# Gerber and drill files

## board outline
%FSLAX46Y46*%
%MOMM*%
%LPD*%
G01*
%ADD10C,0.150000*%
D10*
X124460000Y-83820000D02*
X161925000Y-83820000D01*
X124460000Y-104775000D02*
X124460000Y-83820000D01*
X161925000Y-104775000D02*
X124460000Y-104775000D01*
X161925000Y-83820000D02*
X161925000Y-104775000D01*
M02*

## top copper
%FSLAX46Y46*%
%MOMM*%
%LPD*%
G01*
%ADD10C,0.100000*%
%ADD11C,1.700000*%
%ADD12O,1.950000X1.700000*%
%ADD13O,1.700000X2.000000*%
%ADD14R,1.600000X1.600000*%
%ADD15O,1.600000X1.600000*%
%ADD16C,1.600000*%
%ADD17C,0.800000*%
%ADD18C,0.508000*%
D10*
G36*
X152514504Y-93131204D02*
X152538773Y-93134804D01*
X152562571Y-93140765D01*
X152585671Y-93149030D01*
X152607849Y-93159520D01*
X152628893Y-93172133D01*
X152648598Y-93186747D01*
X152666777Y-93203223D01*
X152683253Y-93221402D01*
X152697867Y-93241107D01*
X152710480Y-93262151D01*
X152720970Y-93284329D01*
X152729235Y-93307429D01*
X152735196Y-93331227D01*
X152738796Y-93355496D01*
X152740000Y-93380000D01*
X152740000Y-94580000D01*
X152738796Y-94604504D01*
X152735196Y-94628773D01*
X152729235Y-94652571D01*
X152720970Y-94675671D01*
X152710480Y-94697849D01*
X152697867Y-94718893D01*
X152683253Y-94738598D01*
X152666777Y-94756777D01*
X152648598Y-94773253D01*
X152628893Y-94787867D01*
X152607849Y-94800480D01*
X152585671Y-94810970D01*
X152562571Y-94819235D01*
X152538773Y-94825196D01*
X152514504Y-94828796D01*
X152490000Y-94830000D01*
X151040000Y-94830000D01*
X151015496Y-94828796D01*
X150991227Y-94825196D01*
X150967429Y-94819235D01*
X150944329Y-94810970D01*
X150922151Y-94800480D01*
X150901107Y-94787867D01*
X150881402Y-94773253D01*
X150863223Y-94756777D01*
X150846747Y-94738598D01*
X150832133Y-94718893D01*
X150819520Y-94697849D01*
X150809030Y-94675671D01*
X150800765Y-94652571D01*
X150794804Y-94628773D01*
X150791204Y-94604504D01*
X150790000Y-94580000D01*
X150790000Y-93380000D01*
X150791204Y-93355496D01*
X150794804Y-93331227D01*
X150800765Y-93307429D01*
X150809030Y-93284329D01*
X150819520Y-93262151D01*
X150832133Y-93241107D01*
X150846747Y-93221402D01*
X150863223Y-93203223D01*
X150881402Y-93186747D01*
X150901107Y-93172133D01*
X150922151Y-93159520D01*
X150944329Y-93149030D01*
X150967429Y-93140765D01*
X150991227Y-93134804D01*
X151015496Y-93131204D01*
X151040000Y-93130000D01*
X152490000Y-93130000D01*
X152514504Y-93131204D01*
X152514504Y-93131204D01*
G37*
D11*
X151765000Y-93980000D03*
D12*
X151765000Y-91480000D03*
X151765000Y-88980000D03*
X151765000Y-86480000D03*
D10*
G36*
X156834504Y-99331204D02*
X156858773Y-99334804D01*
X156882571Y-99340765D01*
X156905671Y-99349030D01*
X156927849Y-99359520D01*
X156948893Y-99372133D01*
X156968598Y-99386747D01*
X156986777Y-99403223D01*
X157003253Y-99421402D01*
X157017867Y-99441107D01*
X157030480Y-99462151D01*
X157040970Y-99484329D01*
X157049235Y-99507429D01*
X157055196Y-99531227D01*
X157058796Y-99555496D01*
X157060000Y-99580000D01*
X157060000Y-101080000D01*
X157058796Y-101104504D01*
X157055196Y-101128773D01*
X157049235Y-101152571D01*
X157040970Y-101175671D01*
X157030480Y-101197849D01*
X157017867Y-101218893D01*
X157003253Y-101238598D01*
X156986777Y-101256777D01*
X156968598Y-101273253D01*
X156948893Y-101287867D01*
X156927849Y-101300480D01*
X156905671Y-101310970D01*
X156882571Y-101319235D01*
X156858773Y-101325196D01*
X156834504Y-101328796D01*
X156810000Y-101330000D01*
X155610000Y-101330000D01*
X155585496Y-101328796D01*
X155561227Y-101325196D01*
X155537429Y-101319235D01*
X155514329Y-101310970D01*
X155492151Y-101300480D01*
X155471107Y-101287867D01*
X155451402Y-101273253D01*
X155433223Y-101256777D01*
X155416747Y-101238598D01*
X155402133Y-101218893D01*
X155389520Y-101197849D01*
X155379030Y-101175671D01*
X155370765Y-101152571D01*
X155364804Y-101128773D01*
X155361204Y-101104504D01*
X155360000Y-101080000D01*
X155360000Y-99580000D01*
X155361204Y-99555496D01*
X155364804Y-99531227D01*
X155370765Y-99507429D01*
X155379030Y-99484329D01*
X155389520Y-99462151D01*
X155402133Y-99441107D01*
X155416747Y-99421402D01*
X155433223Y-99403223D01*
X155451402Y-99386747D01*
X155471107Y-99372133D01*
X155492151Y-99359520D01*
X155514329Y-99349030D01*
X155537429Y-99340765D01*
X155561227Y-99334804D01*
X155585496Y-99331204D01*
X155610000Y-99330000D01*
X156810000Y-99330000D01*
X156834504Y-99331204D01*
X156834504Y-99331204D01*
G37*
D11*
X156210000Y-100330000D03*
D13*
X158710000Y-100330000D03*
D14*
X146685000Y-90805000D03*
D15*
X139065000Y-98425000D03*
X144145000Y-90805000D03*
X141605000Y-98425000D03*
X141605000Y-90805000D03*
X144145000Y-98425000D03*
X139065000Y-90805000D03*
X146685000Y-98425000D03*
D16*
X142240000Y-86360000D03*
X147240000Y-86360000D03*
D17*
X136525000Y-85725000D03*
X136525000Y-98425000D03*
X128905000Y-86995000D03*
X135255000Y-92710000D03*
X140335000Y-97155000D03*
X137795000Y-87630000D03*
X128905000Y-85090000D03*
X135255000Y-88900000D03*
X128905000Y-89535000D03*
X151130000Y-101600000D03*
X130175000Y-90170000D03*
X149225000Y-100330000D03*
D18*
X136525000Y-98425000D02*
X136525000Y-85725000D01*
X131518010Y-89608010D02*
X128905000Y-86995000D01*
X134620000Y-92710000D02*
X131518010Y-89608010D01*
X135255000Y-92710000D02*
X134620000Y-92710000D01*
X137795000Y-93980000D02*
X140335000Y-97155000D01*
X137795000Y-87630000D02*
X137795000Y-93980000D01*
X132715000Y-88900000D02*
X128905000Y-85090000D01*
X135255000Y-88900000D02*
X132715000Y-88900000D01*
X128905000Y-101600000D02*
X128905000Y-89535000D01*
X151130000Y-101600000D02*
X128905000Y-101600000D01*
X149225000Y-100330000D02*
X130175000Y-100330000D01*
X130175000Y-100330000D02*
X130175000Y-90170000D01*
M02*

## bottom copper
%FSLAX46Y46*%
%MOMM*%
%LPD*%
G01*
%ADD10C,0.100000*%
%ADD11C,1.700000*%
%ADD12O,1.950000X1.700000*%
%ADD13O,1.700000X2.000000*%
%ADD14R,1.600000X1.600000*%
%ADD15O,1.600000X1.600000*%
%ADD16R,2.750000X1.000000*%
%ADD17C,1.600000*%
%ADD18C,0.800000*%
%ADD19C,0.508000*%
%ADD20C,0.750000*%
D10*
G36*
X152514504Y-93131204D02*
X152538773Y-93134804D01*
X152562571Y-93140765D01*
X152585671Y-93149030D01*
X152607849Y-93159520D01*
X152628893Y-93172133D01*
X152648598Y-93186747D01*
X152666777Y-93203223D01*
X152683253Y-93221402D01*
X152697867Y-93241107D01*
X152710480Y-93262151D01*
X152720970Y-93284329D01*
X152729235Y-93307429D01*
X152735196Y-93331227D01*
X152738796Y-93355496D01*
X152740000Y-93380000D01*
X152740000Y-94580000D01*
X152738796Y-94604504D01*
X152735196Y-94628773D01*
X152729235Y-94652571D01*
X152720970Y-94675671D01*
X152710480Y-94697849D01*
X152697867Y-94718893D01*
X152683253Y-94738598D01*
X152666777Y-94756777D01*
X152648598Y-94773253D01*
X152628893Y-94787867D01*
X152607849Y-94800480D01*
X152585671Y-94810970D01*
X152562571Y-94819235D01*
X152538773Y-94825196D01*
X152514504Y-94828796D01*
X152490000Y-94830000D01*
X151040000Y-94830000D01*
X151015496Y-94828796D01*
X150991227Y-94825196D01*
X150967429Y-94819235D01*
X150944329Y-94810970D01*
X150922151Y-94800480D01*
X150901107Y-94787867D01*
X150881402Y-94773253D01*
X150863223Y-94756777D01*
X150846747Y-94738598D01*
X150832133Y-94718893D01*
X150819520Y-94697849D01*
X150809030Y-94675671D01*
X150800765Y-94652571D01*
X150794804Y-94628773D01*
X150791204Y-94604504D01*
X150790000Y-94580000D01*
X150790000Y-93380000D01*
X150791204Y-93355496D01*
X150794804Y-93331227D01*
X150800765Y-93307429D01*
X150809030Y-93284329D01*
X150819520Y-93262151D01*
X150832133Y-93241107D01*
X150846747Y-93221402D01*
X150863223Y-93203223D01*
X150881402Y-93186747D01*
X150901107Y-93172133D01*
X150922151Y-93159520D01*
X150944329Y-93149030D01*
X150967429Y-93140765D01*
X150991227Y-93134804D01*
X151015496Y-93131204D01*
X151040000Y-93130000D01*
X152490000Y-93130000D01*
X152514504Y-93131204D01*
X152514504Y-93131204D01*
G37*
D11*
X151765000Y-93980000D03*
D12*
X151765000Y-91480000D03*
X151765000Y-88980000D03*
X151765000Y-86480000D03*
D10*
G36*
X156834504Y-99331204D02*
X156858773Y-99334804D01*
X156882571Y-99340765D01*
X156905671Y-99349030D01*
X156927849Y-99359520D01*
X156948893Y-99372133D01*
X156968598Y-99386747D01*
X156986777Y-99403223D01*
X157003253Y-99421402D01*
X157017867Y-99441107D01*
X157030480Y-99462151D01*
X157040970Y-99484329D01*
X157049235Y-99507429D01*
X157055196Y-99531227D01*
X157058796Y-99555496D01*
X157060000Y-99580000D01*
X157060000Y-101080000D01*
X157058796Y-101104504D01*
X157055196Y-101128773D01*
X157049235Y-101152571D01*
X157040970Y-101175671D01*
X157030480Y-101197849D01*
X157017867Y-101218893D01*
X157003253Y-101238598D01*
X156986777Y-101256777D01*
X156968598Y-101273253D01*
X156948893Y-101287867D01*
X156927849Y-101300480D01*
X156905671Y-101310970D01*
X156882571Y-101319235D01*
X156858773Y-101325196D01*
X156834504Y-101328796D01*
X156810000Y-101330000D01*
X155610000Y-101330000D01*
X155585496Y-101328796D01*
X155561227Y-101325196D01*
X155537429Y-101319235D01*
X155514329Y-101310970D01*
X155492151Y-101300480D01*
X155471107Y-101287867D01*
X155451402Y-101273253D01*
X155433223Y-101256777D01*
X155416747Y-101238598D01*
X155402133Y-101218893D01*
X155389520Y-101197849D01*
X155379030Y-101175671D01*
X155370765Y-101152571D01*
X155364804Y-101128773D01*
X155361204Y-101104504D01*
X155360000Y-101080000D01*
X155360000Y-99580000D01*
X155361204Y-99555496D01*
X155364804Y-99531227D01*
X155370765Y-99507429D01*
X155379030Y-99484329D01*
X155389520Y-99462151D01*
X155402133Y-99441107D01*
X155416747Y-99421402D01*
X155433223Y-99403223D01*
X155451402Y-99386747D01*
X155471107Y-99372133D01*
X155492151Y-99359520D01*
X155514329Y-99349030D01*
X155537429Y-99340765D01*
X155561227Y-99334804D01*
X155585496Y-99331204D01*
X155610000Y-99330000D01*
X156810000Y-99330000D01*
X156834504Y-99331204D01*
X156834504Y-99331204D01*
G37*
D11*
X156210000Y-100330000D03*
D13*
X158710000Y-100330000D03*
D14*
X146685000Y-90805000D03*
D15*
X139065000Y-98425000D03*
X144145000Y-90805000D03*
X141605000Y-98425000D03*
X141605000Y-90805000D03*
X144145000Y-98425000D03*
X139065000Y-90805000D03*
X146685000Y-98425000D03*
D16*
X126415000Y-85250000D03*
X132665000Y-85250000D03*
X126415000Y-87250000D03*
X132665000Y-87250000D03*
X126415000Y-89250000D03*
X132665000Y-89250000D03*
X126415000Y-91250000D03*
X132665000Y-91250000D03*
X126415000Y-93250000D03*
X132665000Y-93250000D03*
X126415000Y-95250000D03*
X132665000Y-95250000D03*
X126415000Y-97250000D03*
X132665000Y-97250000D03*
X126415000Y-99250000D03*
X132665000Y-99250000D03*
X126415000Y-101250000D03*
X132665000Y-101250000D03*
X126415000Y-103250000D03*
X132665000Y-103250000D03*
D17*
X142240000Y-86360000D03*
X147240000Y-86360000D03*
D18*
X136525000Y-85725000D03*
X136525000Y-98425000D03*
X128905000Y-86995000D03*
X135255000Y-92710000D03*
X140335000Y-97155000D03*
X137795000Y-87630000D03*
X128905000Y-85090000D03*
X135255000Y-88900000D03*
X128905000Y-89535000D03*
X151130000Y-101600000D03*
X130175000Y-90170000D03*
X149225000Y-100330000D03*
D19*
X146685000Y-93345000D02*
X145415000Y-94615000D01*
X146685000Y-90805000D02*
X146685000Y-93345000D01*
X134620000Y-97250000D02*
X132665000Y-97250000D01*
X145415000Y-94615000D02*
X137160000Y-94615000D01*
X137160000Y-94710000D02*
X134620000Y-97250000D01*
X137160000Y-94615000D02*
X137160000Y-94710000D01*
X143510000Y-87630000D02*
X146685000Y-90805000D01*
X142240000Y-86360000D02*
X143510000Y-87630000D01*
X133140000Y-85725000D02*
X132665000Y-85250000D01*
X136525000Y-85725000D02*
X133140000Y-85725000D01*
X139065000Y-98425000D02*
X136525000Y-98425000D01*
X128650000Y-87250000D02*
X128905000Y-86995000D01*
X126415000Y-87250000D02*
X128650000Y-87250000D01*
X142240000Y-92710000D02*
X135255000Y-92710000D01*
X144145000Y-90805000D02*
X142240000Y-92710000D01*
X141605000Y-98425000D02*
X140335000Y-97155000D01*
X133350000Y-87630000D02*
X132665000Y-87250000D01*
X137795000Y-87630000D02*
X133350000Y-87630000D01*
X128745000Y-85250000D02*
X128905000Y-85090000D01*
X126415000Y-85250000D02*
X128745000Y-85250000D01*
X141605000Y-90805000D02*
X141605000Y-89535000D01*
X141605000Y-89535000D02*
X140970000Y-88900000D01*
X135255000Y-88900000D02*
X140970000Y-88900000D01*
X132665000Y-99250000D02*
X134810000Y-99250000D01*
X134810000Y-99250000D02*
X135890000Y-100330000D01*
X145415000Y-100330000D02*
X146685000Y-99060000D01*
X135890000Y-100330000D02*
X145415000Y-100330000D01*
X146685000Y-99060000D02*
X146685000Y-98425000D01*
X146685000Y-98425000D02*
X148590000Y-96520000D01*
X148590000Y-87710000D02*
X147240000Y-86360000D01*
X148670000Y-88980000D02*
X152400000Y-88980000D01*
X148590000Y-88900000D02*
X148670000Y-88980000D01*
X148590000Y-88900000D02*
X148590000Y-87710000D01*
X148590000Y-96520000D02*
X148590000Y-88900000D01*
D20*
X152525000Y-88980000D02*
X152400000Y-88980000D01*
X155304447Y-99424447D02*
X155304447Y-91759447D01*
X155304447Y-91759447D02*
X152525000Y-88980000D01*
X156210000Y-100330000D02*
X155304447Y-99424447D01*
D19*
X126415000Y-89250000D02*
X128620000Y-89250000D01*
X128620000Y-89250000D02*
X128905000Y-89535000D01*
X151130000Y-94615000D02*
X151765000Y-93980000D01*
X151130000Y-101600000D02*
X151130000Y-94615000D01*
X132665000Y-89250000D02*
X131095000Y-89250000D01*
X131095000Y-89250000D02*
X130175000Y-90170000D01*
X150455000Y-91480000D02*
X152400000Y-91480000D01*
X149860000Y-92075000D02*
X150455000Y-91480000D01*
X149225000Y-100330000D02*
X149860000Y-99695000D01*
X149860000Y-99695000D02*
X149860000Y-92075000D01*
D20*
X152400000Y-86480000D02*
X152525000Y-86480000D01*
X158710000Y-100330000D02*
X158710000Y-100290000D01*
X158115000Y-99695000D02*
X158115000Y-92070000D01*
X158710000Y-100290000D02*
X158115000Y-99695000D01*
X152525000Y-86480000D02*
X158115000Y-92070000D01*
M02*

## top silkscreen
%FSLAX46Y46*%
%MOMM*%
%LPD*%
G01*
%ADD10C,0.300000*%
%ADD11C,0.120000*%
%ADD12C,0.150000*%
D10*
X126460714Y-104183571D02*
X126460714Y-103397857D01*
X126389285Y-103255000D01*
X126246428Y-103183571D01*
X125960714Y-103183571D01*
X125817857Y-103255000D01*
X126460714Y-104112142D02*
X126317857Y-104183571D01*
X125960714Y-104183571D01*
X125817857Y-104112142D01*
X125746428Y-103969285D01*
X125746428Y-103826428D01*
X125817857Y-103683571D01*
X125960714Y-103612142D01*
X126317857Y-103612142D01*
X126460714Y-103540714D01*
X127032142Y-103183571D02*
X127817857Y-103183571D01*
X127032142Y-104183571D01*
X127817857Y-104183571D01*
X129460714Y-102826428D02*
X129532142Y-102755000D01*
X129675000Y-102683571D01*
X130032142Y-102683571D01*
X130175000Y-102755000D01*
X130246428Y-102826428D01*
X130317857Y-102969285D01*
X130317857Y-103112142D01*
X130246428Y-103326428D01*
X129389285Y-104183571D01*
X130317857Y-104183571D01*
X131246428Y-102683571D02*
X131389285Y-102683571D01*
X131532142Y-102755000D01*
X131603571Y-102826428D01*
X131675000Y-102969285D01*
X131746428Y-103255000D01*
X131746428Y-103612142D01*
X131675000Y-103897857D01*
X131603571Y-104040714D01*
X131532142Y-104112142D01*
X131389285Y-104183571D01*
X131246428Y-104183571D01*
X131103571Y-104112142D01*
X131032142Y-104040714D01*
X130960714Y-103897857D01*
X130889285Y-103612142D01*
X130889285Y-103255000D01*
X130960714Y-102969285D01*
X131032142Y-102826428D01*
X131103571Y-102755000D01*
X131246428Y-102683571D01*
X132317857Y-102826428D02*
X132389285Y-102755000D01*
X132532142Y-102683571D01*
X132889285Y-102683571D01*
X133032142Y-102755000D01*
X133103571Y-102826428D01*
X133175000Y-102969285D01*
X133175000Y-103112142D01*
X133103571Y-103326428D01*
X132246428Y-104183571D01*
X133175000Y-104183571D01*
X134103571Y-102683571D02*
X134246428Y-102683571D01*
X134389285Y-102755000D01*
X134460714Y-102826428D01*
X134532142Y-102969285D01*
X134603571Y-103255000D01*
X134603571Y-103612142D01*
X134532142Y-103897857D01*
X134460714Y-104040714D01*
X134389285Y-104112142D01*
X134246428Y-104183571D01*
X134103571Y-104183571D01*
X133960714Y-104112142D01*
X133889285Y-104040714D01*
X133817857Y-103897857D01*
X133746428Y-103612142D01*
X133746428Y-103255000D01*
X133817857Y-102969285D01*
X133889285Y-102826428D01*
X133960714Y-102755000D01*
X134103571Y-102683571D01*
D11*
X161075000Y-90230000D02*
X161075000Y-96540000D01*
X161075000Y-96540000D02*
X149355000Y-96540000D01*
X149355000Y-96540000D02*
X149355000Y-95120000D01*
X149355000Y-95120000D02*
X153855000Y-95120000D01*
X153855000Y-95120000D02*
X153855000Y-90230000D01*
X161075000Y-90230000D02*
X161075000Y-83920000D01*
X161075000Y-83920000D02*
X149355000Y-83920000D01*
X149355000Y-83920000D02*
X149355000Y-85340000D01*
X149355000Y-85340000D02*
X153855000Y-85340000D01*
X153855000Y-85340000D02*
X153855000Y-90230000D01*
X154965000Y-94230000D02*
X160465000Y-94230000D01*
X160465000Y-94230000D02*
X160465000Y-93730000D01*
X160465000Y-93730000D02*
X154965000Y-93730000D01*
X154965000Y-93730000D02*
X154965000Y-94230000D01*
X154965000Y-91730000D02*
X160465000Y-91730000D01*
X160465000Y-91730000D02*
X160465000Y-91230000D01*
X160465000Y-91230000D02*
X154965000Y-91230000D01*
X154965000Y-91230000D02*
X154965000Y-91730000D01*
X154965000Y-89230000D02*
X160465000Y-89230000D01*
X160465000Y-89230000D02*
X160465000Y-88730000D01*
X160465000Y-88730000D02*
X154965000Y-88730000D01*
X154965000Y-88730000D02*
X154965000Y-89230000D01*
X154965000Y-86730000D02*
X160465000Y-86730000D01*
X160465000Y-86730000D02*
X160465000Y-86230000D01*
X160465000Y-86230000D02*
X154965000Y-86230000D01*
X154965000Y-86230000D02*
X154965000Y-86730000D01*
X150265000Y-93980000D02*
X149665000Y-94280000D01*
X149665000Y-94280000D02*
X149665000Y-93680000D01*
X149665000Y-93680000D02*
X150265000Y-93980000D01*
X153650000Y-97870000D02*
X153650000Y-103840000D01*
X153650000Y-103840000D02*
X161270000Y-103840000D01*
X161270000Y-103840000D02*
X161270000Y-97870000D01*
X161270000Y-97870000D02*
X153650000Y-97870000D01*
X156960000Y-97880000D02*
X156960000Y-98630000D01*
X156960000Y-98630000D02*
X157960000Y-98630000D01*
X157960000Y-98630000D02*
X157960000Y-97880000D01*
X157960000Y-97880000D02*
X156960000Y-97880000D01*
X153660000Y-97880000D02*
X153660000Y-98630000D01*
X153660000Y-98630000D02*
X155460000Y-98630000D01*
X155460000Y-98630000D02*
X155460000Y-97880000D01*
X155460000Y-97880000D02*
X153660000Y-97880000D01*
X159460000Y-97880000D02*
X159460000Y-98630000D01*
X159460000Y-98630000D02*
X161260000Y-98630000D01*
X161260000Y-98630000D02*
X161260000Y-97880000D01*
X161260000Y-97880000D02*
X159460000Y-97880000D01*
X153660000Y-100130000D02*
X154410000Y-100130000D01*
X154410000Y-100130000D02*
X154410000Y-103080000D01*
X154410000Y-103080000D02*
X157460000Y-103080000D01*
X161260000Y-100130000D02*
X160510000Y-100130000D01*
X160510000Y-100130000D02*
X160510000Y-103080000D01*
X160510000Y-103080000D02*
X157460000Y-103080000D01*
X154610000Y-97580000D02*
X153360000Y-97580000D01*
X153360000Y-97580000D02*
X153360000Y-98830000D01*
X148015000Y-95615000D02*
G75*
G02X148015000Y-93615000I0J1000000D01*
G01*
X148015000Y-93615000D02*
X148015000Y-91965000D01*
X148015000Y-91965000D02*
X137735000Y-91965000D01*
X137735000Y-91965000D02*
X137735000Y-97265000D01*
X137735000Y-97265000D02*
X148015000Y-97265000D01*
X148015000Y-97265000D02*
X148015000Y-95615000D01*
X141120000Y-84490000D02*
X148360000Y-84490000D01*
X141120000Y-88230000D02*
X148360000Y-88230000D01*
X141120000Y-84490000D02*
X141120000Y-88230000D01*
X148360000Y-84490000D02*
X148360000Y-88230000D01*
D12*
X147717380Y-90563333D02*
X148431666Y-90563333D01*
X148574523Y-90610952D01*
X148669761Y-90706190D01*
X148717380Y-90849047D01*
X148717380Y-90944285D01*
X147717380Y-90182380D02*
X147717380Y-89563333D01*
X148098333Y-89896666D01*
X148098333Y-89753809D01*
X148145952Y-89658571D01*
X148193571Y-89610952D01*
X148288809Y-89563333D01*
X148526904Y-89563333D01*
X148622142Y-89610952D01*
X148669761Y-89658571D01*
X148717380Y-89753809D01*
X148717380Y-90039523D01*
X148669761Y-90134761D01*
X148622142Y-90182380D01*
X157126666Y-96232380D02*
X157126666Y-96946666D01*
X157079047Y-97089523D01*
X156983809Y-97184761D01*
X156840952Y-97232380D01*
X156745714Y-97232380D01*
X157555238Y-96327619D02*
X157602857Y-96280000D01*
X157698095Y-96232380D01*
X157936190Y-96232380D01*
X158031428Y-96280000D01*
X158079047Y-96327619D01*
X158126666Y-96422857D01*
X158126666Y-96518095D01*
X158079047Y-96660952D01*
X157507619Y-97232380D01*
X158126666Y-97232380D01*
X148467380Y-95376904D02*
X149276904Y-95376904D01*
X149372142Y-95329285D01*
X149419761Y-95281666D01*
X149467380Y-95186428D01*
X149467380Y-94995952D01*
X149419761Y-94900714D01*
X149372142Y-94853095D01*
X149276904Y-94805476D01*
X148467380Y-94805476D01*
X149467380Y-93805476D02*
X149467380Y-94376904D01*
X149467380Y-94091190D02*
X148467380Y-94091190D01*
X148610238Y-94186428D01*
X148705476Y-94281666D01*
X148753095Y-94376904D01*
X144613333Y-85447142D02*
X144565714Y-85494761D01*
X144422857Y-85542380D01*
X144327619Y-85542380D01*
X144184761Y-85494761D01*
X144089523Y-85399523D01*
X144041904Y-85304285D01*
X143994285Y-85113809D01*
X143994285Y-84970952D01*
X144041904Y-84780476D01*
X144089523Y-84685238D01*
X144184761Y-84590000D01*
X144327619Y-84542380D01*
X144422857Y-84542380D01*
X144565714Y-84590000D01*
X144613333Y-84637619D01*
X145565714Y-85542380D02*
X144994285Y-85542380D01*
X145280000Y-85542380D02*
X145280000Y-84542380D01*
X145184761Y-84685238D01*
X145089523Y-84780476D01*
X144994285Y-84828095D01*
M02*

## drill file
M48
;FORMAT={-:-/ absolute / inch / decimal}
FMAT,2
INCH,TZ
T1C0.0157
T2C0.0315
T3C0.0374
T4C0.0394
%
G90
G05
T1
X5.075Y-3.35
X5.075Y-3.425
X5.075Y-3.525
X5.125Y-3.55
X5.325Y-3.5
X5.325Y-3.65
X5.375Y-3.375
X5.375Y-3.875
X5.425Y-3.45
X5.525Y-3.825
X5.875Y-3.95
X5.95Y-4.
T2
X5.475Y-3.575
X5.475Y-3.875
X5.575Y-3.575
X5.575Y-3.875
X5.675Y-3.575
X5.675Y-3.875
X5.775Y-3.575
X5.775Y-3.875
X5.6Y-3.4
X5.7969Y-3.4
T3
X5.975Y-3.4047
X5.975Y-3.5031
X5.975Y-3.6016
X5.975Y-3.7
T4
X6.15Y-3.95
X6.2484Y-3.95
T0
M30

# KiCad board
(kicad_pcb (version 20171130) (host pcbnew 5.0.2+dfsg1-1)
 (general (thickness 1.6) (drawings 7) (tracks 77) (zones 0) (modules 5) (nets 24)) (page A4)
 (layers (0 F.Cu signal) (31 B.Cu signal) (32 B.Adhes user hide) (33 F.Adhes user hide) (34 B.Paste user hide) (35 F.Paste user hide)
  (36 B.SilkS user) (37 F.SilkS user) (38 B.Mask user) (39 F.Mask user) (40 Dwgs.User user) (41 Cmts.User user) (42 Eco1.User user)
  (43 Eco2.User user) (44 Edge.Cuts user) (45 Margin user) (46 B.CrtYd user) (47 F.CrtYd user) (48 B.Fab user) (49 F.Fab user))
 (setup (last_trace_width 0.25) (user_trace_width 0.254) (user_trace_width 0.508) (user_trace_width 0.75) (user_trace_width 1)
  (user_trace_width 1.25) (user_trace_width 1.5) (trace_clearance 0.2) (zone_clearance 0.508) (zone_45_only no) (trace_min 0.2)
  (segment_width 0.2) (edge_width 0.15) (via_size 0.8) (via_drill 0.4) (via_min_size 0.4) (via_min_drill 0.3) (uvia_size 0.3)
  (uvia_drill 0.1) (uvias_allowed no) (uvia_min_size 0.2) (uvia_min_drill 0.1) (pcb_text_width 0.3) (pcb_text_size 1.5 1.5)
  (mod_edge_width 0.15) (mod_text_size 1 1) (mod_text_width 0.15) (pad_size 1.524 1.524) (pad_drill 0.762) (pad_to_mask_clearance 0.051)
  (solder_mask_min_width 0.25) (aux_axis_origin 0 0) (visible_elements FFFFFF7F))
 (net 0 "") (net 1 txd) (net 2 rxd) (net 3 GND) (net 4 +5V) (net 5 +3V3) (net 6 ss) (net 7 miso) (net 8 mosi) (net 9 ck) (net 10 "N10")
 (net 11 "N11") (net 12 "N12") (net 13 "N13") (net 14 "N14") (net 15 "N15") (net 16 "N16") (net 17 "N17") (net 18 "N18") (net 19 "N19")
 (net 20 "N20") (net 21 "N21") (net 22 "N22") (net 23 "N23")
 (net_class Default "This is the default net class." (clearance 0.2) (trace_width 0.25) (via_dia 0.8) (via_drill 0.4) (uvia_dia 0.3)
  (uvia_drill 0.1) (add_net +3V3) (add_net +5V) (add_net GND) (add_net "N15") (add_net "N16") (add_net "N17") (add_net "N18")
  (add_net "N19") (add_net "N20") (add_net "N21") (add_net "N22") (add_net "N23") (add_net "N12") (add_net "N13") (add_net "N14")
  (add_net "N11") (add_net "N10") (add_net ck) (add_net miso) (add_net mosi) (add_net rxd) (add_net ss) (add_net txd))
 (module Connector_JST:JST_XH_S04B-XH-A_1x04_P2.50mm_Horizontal (layer F.Cu) (at 151.765 93.98 90)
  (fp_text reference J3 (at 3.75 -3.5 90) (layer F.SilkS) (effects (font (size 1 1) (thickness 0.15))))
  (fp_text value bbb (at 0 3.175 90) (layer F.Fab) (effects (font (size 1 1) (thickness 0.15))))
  (fp_line (start 3.75 9.31) (end -2.56 9.31) (layer F.SilkS) (width 0.12))
  (fp_line (start -2.56 9.31) (end -2.56 -2.41) (layer F.SilkS) (width 0.12))
  (fp_line (start -2.56 -2.41) (end -1.14 -2.41) (layer F.SilkS) (width 0.12))
  (fp_line (start -1.14 -2.41) (end -1.14 2.09) (layer F.SilkS) (width 0.12))
  (fp_line (start -1.14 2.09) (end 3.75 2.09) (layer F.SilkS) (width 0.12))
  (fp_line (start 3.75 9.31) (end 10.06 9.31) (layer F.SilkS) (width 0.12))
  (fp_line (start 10.06 9.31) (end 10.06 -2.41) (layer F.SilkS) (width 0.12))
  (fp_line (start 10.06 -2.41) (end 8.64 -2.41) (layer F.SilkS) (width 0.12))
  (fp_line (start 8.64 -2.41) (end 8.64 2.09) (layer F.SilkS) (width 0.12))
  (fp_line (start 8.64 2.09) (end 3.75 2.09) (layer F.SilkS) (width 0.12))
  (fp_line (start -0.25 3.2) (end -0.25 8.7) (layer F.SilkS) (width 0.12))
  (fp_line (start -0.25 8.7) (end 0.25 8.7) (layer F.SilkS) (width 0.12))
  (fp_line (start 0.25 8.7) (end 0.25 3.2) (layer F.SilkS) (width 0.12))
  (fp_line (start 0.25 3.2) (end -0.25 3.2) (layer F.SilkS) (width 0.12))
  (fp_line (start 2.25 3.2) (end 2.25 8.7) (layer F.SilkS) (width 0.12))
  (fp_line (start 2.25 8.7) (end 2.75 8.7) (layer F.SilkS) (width 0.12))
  (fp_line (start 2.75 8.7) (end 2.75 3.2) (layer F.SilkS) (width 0.12))
  (fp_line (start 2.75 3.2) (end 2.25 3.2) (layer F.SilkS) (width 0.12))
  (fp_line (start 4.75 3.2) (end 4.75 8.7) (layer F.SilkS) (width 0.12))
  (fp_line (start 4.75 8.7) (end 5.25 8.7) (layer F.SilkS) (width 0.12))
  (fp_line (start 5.25 8.7) (end 5.25 3.2) (layer F.SilkS) (width 0.12))
  (fp_line (start 5.25 3.2) (end 4.75 3.2) (layer F.SilkS) (width 0.12))
  (fp_line (start 7.25 3.2) (end 7.25 8.7) (layer F.SilkS) (width 0.12))
  (fp_line (start 7.25 8.7) (end 7.75 8.7) (layer F.SilkS) (width 0.12))
  (fp_line (start 7.75 8.7) (end 7.75 3.2) (layer F.SilkS) (width 0.12))
  (fp_line (start 7.75 3.2) (end 7.25 3.2) (layer F.SilkS) (width 0.12))
  (fp_line (start 0 -1.5) (end -0.3 -2.1) (layer F.SilkS) (width 0.12))
  (fp_line (start -0.3 -2.1) (end 0.3 -2.1) (layer F.SilkS) (width 0.12))
  (fp_line (start 0.3 -2.1) (end 0 -1.5) (layer F.SilkS) (width 0.12))
  (pad 1 thru_hole roundrect (at 0 0 90) (size 1.7 1.95) (drill 0.95) (layers *.Cu *.Mask) (roundrect_rratio 0.147059) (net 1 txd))
  (pad 2 thru_hole oval (at 2.5 0 90) (size 1.7 1.95) (drill 0.95) (layers *.Cu *.Mask) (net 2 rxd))
  (pad 3 thru_hole oval (at 5 0 90) (size 1.7 1.95) (drill 0.95) (layers *.Cu *.Mask) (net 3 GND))
  (pad 4 thru_hole oval (at 7.5 0 90) (size 1.7 1.95) (drill 0.95) (layers *.Cu *.Mask) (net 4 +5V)))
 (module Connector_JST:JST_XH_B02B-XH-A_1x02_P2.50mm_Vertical (layer F.Cu) (at 156.21 100.33)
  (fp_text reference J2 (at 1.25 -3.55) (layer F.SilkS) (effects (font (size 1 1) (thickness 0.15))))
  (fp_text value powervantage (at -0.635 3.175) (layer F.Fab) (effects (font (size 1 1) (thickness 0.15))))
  (fp_line (start -2.56 -2.46) (end -2.56 3.51) (layer F.SilkS) (width 0.12))
  (fp_line (start -2.56 3.51) (end 5.06 3.51) (layer F.SilkS) (width 0.12))
  (fp_line (start 5.06 3.51) (end 5.06 -2.46) (layer F.SilkS) (width 0.12))
  (fp_line (start 5.06 -2.46) (end -2.56 -2.46) (layer F.SilkS) (width 0.12))
  (fp_line (start 0.75 -2.45) (end 0.75 -1.7) (layer F.SilkS) (width 0.12))
  (fp_line (start 0.75 -1.7) (end 1.75 -1.7) (layer F.SilkS) (width 0.12))
  (fp_line (start 1.75 -1.7) (end 1.75 -2.45) (layer F.SilkS) (width 0.12))
  (fp_line (start 1.75 -2.45) (end 0.75 -2.45) (layer F.SilkS) (width 0.12))
  (fp_line (start -2.55 -2.45) (end -2.55 -1.7) (layer F.SilkS) (width 0.12))
  (fp_line (start -2.55 -1.7) (end -0.75 -1.7) (layer F.SilkS) (width 0.12))
  (fp_line (start -0.75 -1.7) (end -0.75 -2.45) (layer F.SilkS) (width 0.12))
  (fp_line (start -0.75 -2.45) (end -2.55 -2.45) (layer F.SilkS) (width 0.12))
  (fp_line (start 3.25 -2.45) (end 3.25 -1.7) (layer F.SilkS) (width 0.12))
  (fp_line (start 3.25 -1.7) (end 5.05 -1.7) (layer F.SilkS) (width 0.12))
  (fp_line (start 5.05 -1.7) (end 5.05 -2.45) (layer F.SilkS) (width 0.12))
  (fp_line (start 5.05 -2.45) (end 3.25 -2.45) (layer F.SilkS) (width 0.12))
  (fp_line (start -2.55 -0.2) (end -1.8 -0.2) (layer F.SilkS) (width 0.12))
  (fp_line (start -1.8 -0.2) (end -1.8 2.75) (layer F.SilkS) (width 0.12))
  (fp_line (start -1.8 2.75) (end 1.25 2.75) (layer F.SilkS) (width 0.12))
  (fp_line (start 5.05 -0.2) (end 4.3 -0.2) (layer F.SilkS) (width 0.12))
  (fp_line (start 4.3 -0.2) (end 4.3 2.75) (layer F.SilkS) (width 0.12))
  (fp_line (start 4.3 2.75) (end 1.25 2.75) (layer F.SilkS) (width 0.12))
  (fp_line (start -1.6 -2.75) (end -2.85 -2.75) (layer F.SilkS) (width 0.12))
  (fp_line (start -2.85 -2.75) (end -2.85 -1.5) (layer F.SilkS) (width 0.12))
  (pad 1 thru_hole roundrect (at 0 0) (size 1.7 2) (drill 1) (layers *.Cu *.Mask) (roundrect_rratio 0.147059) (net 3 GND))
  (pad 2 thru_hole oval (at 2.5 0) (size 1.7 2) (drill 1) (layers *.Cu *.Mask) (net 4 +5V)))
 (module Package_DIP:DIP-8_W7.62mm (layer F.Cu) (at 146.685 90.805 270)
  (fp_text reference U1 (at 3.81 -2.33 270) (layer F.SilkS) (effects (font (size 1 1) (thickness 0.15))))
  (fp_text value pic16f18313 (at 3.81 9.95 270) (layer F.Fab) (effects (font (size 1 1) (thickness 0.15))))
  (fp_arc (start 3.81 -1.33) (end 2.81 -1.33) (angle -180) (layer F.SilkS) (width 0.12))
  (fp_line (start 2.81 -1.33) (end 1.16 -1.33) (layer F.SilkS) (width 0.12))
  (fp_line (start 1.16 -1.33) (end 1.16 8.95) (layer F.SilkS) (width 0.12))
  (fp_line (start 1.16 8.95) (end 6.46 8.95) (layer F.SilkS) (width 0.12))
  (fp_line (start 6.46 8.95) (end 6.46 -1.33) (layer F.SilkS) (width 0.12))
  (fp_line (start 6.46 -1.33) (end 4.81 -1.33) (layer F.SilkS) (width 0.12))
  (pad 1 thru_hole rect (at 0 0 270) (size 1.6 1.6) (drill 0.8) (layers *.Cu *.Mask) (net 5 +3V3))
  (pad 5 thru_hole oval (at 7.62 7.62 270) (size 1.6 1.6) (drill 0.8) (layers *.Cu *.Mask) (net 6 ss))
  (pad 2 thru_hole oval (at 0 2.54 270) (size 1.6 1.6) (drill 0.8) (layers *.Cu *.Mask) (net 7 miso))
  (pad 6 thru_hole oval (at 7.62 5.08 270) (size 1.6 1.6) (drill 0.8) (layers *.Cu *.Mask) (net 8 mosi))
  (pad 3 thru_hole oval (at 0 5.08 270) (size 1.6 1.6) (drill 0.8) (layers *.Cu *.Mask) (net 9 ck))
  (pad 7 thru_hole oval (at 7.62 2.54 270) (size 1.6 1.6) (drill 0.8) (layers *.Cu *.Mask) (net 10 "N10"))
  (pad 4 thru_hole oval (at 0 7.62 270) (size 1.6 1.6) (drill 0.8) (layers *.Cu *.Mask) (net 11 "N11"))
  (pad 8 thru_hole oval (at 7.62 0 270) (size 1.6 1.6) (drill 0.8) (layers *.Cu *.Mask) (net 3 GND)))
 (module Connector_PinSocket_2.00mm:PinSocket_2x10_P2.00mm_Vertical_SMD (layer B.Cu) (at 129.54 94.25 180)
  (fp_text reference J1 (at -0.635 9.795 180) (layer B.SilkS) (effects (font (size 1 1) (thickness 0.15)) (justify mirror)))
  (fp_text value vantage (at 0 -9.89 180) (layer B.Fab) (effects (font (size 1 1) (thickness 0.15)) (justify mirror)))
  (pad 1 smd rect (at 3.125 9 180) (size 2.75 1) (layers B.Cu B.Paste B.Mask) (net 9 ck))
  (pad 2 smd rect (at -3.125 9 180) (size 2.75 1) (layers B.Cu B.Paste B.Mask) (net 6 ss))
  (pad 3 smd rect (at 3.125 7 180) (size 2.75 1) (layers B.Cu B.Paste B.Mask) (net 7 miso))
  (pad 4 smd rect (at -3.125 7 180) (size 2.75 1) (layers B.Cu B.Paste B.Mask) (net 8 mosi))
  (pad 5 smd rect (at 3.125 5 180) (size 2.75 1) (layers B.Cu B.Paste B.Mask) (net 1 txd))
  (pad 6 smd rect (at -3.125 5 180) (size 2.75 1) (layers B.Cu B.Paste B.Mask) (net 2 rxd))
  (pad 7 smd rect (at 3.125 3 180) (size 2.75 1) (layers B.Cu B.Paste B.Mask) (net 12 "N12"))
  (pad 8 smd rect (at -3.125 3 180) (size 2.75 1) (layers B.Cu B.Paste B.Mask) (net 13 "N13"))
  (pad 9 smd rect (at 3.125 1 180) (size 2.75 1) (layers B.Cu B.Paste B.Mask) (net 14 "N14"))
  (pad 10 smd rect (at -3.125 1 180) (size 2.75 1) (layers B.Cu B.Paste B.Mask) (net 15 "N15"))
  (pad 11 smd rect (at 3.125 -1 180) (size 2.75 1) (layers B.Cu B.Paste B.Mask) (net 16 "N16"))
  (pad 12 smd rect (at -3.125 -1 180) (size 2.75 1) (layers B.Cu B.Paste B.Mask) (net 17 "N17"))
  (pad 13 smd rect (at 3.125 -3 180) (size 2.75 1) (layers B.Cu B.Paste B.Mask) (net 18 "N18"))
  (pad 14 smd rect (at -3.125 -3 180) (size 2.75 1) (layers B.Cu B.Paste B.Mask) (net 5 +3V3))
  (pad 15 smd rect (at 3.125 -5 180) (size 2.75 1) (layers B.Cu B.Paste B.Mask) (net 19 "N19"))
  (pad 16 smd rect (at -3.125 -5 180) (size 2.75 1) (layers B.Cu B.Paste B.Mask) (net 3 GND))
  (pad 17 smd rect (at 3.125 -7 180) (size 2.75 1) (layers B.Cu B.Paste B.Mask) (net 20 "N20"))
  (pad 18 smd rect (at -3.125 -7 180) (size 2.75 1) (layers B.Cu B.Paste B.Mask) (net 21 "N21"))
  (pad 19 smd rect (at 3.125 -9 180) (size 2.75 1) (layers B.Cu B.Paste B.Mask) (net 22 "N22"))
  (pad 20 smd rect (at -3.125 -9 180) (size 2.75 1) (layers B.Cu B.Paste B.Mask) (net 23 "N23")))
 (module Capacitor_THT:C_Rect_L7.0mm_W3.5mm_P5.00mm (layer F.Cu) (at 142.24 86.36)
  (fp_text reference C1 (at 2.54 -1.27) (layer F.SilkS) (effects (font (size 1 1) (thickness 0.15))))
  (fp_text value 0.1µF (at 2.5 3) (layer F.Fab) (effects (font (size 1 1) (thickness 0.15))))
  (fp_line (start -1.12 -1.87) (end 6.12 -1.87) (layer F.SilkS) (width 0.12))
  (fp_line (start -1.12 1.87) (end 6.12 1.87) (layer F.SilkS) (width 0.12))
  (fp_line (start -1.12 -1.87) (end -1.12 1.87) (layer F.SilkS) (width 0.12))
  (fp_line (start 6.12 -1.87) (end 6.12 1.87) (layer F.SilkS) (width 0.12))
  (pad 1 thru_hole circle (at 0 0) (size 1.6 1.6) (drill 0.8) (layers *.Cu *.Mask) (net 5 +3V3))
  (pad 2 thru_hole circle (at 5 0) (size 1.6 1.6) (drill 0.8) (layers *.Cu *.Mask) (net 3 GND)))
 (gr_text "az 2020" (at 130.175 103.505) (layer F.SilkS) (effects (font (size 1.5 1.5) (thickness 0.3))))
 (gr_line (start 124.46 83.82) (end 161.925 83.82) (layer Edge.Cuts) (width 0.15))
 (gr_line (start 124.46 104.775) (end 124.46 83.82) (layer Edge.Cuts) (width 0.15))
 (gr_line (start 161.925 104.775) (end 124.46 104.775) (layer Edge.Cuts) (width 0.15))
 (gr_line (start 161.925 83.82) (end 161.925 104.775) (layer Edge.Cuts) (width 0.15))
 (segment (start 146.685 93.345) (end 145.415 94.615) (width 0.508) (layer B.Cu) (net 5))
 (segment (start 146.685 90.805) (end 146.685 93.345) (width 0.508) (layer B.Cu) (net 5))
 (segment (start 134.62 97.25) (end 132.665 97.25) (width 0.508) (layer B.Cu) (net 5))
 (segment (start 145.415 94.615) (end 137.16 94.615) (width 0.508) (layer B.Cu) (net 5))
 (segment (start 137.16 94.71) (end 134.62 97.25) (width 0.508) (layer B.Cu) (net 5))
 (segment (start 137.16 94.615) (end 137.16 94.71) (width 0.508) (layer B.Cu) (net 5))
 (segment (start 143.51 87.63) (end 146.685 90.805) (width 0.508) (layer B.Cu) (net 5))
 (segment (start 142.24 86.36) (end 143.51 87.63) (width 0.508) (layer B.Cu) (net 5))
 (segment (start 133.14 85.725) (end 132.665 85.25) (width 0.508) (layer B.Cu) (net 6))
 (via (at 136.525 85.725) (size 0.8) (drill 0.4) (layers F.Cu B.Cu) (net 6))
 (segment (start 136.525 85.725) (end 133.14 85.725) (width 0.508) (layer B.Cu) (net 6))
 (segment (start 136.525 98.425) (end 136.525 85.725) (width 0.508) (layer F.Cu) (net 6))
 (via (at 136.525 98.425) (size 0.8) (drill 0.4) (layers F.Cu B.Cu) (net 6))
 (segment (start 139.065 98.425) (end 136.525 98.425) (width 0.508) (layer B.Cu) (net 6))
 (via (at 128.905 86.995) (size 0.8) (drill 0.4) (layers F.Cu B.Cu) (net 7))
 (segment (start 128.65 87.25) (end 128.905 86.995) (width 0.508) (layer B.Cu) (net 7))
 (segment (start 126.415 87.25) (end 128.65 87.25) (width 0.508) (layer B.Cu) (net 7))
 (segment (start 131.51801 89.60801) (end 128.905 86.995) (width 0.508) (layer F.Cu) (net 7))
 (via (at 135.255 92.71) (size 0.8) (drill 0.4) (layers F.Cu B.Cu) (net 7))
 (segment (start 134.62 92.71) (end 131.51801 89.60801) (width 0.508) (layer F.Cu) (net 7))
 (segment (start 135.255 92.71) (end 134.62 92.71) (width 0.508) (layer F.Cu) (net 7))
 (segment (start 142.24 92.71) (end 135.255 92.71) (width 0.508) (layer B.Cu) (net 7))
 (segment (start 144.145 90.805) (end 142.24 92.71) (width 0.508) (layer B.Cu) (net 7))
 (segment (start 141.605 98.425) (end 140.335 97.155) (width 0.508) (layer B.Cu) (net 8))
 (via (at 140.335 97.155) (size 0.8) (drill 0.4) (layers F.Cu B.Cu) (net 8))
 (segment (start 137.795 93.98) (end 140.335 97.155) (width 0.508) (layer F.Cu) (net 8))
 (segment (start 137.795 87.63) (end 137.795 93.98) (width 0.508) (layer F.Cu) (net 8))
 (segment (start 133.35 87.63) (end 132.665 87.25) (width 0.508) (layer B.Cu) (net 8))
 (via (at 137.795 87.63) (size 0.8) (drill 0.4) (layers F.Cu B.Cu) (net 8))
 (segment (start 137.795 87.63) (end 133.35 87.63) (width 0.508) (layer B.Cu) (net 8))
 (segment (start 128.745 85.25) (end 128.905 85.09) (width 0.508) (layer B.Cu) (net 9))
 (via (at 128.905 85.09) (size 0.8) (drill 0.4) (layers F.Cu B.Cu) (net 9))
 (segment (start 126.415 85.25) (end 128.745 85.25) (width 0.508) (layer B.Cu) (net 9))
 (segment (start 132.715 88.9) (end 128.905 85.09) (width 0.508) (layer F.Cu) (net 9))
 (via (at 135.255 88.9) (size 0.8) (drill 0.4) (layers F.Cu B.Cu) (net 9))
 (segment (start 135.255 88.9) (end 132.715 88.9) (width 0.508) (layer F.Cu) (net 9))
 (segment (start 141.605 90.805) (end 141.605 89.535) (width 0.508) (layer B.Cu) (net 9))
 (segment (start 141.605 89.535) (end 140.97 88.9) (width 0.508) (layer B.Cu) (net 9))
 (segment (start 135.255 88.9) (end 140.97 88.9) (width 0.508) (layer B.Cu) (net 9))
 (segment (start 132.665 99.25) (end 134.81 99.25) (width 0.508) (layer B.Cu) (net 3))
 (segment (start 134.81 99.25) (end 135.89 100.33) (width 0.508) (layer B.Cu) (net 3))
 (segment (start 145.415 100.33) (end 146.685 99.06) (width 0.508) (layer B.Cu) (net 3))
 (segment (start 135.89 100.33) (end 145.415 100.33) (width 0.508) (layer B.Cu) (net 3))
 (segment (start 146.685 99.06) (end 146.685 98.425) (width 0.508) (layer B.Cu) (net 3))
 (segment (start 146.685 98.425) (end 148.59 96.52) (width 0.508) (layer B.Cu) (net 3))
 (segment (start 148.59 87.71) (end 147.24 86.36) (width 0.508) (layer B.Cu) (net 3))
 (segment (start 148.67 88.98) (end 152.4 88.98) (width 0.508) (layer B.Cu) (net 3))
 (segment (start 148.59 88.9) (end 148.67 88.98) (width 0.508) (layer B.Cu) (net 3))
 (segment (start 148.59 88.9) (end 148.59 87.71) (width 0.508) (layer B.Cu) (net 3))
 (segment (start 148.59 96.52) (end 148.59 88.9) (width 0.508) (layer B.Cu) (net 3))
 (segment (start 152.525 88.98) (end 152.4 88.98) (width 0.75) (layer B.Cu) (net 3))
 (segment (start 155.304447 99.424447) (end 155.304447 91.759447) (width 0.75) (layer B.Cu) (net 3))
 (segment (start 155.304447 91.759447) (end 152.525 88.98) (width 0.75) (layer B.Cu) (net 3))
 (segment (start 156.21 100.33) (end 155.304447 99.424447) (width 0.75) (layer B.Cu) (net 3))
 (via (at 128.905 89.535) (size 0.8) (drill 0.4) (layers F.Cu B.Cu) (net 1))
 (segment (start 126.415 89.25) (end 128.62 89.25) (width 0.508) (layer B.Cu) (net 1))
 (segment (start 128.62 89.25) (end 128.905 89.535) (width 0.508) (layer B.Cu) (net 1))
 (segment (start 128.905 101.6) (end 128.905 89.535) (width 0.508) (layer F.Cu) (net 1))
 (segment (start 151.13 101.6) (end 128.905 101.6) (width 0.508) (layer F.Cu) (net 1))
 (via (at 151.13 101.6) (size 0.8) (drill 0.4) (layers F.Cu B.Cu) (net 1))
 (segment (start 151.13 94.615) (end 151.765 93.98) (width 0.508) (layer B.Cu) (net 1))
 (segment (start 151.13 101.6) (end 151.13 94.615) (width 0.508) (layer B.Cu) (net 1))
 (via (at 130.175 90.17) (size 0.8) (drill 0.4) (layers F.Cu B.Cu) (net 2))
 (segment (start 132.665 89.25) (end 131.095 89.25) (width 0.508) (layer B.Cu) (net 2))
 (segment (start 131.095 89.25) (end 130.175 90.17) (width 0.508) (layer B.Cu) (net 2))
 (segment (start 149.225 100.33) (end 130.175 100.33) (width 0.508) (layer F.Cu) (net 2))
 (via (at 149.225 100.33) (size 0.8) (drill 0.4) (layers F.Cu B.Cu) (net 2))
 (segment (start 130.175 100.33) (end 130.175 90.17) (width 0.508) (layer F.Cu) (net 2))
 (segment (start 150.455 91.48) (end 152.4 91.48) (width 0.508) (layer B.Cu) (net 2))
 (segment (start 149.86 92.075) (end 150.455 91.48) (width 0.508) (layer B.Cu) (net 2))
 (segment (start 149.225 100.33) (end 149.86 99.695) (width 0.508) (layer B.Cu) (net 2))
 (segment (start 149.86 99.695) (end 149.86 92.075) (width 0.508) (layer B.Cu) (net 2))
 (segment (start 152.4 86.48) (end 152.525 86.48) (width 0.75) (layer B.Cu) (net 4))
 (segment (start 158.71 100.33) (end 158.71 100.29) (width 0.75) (layer B.Cu) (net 4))
 (segment (start 158.115 99.695) (end 158.115 92.07) (width 0.75) (layer B.Cu) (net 4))
 (segment (start 158.71 100.29) (end 158.115 99.695) (width 0.75) (layer B.Cu) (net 4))
 (segment (start 152.525 86.48) (end 158.115 92.07) (width 0.75) (layer B.Cu) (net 4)))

